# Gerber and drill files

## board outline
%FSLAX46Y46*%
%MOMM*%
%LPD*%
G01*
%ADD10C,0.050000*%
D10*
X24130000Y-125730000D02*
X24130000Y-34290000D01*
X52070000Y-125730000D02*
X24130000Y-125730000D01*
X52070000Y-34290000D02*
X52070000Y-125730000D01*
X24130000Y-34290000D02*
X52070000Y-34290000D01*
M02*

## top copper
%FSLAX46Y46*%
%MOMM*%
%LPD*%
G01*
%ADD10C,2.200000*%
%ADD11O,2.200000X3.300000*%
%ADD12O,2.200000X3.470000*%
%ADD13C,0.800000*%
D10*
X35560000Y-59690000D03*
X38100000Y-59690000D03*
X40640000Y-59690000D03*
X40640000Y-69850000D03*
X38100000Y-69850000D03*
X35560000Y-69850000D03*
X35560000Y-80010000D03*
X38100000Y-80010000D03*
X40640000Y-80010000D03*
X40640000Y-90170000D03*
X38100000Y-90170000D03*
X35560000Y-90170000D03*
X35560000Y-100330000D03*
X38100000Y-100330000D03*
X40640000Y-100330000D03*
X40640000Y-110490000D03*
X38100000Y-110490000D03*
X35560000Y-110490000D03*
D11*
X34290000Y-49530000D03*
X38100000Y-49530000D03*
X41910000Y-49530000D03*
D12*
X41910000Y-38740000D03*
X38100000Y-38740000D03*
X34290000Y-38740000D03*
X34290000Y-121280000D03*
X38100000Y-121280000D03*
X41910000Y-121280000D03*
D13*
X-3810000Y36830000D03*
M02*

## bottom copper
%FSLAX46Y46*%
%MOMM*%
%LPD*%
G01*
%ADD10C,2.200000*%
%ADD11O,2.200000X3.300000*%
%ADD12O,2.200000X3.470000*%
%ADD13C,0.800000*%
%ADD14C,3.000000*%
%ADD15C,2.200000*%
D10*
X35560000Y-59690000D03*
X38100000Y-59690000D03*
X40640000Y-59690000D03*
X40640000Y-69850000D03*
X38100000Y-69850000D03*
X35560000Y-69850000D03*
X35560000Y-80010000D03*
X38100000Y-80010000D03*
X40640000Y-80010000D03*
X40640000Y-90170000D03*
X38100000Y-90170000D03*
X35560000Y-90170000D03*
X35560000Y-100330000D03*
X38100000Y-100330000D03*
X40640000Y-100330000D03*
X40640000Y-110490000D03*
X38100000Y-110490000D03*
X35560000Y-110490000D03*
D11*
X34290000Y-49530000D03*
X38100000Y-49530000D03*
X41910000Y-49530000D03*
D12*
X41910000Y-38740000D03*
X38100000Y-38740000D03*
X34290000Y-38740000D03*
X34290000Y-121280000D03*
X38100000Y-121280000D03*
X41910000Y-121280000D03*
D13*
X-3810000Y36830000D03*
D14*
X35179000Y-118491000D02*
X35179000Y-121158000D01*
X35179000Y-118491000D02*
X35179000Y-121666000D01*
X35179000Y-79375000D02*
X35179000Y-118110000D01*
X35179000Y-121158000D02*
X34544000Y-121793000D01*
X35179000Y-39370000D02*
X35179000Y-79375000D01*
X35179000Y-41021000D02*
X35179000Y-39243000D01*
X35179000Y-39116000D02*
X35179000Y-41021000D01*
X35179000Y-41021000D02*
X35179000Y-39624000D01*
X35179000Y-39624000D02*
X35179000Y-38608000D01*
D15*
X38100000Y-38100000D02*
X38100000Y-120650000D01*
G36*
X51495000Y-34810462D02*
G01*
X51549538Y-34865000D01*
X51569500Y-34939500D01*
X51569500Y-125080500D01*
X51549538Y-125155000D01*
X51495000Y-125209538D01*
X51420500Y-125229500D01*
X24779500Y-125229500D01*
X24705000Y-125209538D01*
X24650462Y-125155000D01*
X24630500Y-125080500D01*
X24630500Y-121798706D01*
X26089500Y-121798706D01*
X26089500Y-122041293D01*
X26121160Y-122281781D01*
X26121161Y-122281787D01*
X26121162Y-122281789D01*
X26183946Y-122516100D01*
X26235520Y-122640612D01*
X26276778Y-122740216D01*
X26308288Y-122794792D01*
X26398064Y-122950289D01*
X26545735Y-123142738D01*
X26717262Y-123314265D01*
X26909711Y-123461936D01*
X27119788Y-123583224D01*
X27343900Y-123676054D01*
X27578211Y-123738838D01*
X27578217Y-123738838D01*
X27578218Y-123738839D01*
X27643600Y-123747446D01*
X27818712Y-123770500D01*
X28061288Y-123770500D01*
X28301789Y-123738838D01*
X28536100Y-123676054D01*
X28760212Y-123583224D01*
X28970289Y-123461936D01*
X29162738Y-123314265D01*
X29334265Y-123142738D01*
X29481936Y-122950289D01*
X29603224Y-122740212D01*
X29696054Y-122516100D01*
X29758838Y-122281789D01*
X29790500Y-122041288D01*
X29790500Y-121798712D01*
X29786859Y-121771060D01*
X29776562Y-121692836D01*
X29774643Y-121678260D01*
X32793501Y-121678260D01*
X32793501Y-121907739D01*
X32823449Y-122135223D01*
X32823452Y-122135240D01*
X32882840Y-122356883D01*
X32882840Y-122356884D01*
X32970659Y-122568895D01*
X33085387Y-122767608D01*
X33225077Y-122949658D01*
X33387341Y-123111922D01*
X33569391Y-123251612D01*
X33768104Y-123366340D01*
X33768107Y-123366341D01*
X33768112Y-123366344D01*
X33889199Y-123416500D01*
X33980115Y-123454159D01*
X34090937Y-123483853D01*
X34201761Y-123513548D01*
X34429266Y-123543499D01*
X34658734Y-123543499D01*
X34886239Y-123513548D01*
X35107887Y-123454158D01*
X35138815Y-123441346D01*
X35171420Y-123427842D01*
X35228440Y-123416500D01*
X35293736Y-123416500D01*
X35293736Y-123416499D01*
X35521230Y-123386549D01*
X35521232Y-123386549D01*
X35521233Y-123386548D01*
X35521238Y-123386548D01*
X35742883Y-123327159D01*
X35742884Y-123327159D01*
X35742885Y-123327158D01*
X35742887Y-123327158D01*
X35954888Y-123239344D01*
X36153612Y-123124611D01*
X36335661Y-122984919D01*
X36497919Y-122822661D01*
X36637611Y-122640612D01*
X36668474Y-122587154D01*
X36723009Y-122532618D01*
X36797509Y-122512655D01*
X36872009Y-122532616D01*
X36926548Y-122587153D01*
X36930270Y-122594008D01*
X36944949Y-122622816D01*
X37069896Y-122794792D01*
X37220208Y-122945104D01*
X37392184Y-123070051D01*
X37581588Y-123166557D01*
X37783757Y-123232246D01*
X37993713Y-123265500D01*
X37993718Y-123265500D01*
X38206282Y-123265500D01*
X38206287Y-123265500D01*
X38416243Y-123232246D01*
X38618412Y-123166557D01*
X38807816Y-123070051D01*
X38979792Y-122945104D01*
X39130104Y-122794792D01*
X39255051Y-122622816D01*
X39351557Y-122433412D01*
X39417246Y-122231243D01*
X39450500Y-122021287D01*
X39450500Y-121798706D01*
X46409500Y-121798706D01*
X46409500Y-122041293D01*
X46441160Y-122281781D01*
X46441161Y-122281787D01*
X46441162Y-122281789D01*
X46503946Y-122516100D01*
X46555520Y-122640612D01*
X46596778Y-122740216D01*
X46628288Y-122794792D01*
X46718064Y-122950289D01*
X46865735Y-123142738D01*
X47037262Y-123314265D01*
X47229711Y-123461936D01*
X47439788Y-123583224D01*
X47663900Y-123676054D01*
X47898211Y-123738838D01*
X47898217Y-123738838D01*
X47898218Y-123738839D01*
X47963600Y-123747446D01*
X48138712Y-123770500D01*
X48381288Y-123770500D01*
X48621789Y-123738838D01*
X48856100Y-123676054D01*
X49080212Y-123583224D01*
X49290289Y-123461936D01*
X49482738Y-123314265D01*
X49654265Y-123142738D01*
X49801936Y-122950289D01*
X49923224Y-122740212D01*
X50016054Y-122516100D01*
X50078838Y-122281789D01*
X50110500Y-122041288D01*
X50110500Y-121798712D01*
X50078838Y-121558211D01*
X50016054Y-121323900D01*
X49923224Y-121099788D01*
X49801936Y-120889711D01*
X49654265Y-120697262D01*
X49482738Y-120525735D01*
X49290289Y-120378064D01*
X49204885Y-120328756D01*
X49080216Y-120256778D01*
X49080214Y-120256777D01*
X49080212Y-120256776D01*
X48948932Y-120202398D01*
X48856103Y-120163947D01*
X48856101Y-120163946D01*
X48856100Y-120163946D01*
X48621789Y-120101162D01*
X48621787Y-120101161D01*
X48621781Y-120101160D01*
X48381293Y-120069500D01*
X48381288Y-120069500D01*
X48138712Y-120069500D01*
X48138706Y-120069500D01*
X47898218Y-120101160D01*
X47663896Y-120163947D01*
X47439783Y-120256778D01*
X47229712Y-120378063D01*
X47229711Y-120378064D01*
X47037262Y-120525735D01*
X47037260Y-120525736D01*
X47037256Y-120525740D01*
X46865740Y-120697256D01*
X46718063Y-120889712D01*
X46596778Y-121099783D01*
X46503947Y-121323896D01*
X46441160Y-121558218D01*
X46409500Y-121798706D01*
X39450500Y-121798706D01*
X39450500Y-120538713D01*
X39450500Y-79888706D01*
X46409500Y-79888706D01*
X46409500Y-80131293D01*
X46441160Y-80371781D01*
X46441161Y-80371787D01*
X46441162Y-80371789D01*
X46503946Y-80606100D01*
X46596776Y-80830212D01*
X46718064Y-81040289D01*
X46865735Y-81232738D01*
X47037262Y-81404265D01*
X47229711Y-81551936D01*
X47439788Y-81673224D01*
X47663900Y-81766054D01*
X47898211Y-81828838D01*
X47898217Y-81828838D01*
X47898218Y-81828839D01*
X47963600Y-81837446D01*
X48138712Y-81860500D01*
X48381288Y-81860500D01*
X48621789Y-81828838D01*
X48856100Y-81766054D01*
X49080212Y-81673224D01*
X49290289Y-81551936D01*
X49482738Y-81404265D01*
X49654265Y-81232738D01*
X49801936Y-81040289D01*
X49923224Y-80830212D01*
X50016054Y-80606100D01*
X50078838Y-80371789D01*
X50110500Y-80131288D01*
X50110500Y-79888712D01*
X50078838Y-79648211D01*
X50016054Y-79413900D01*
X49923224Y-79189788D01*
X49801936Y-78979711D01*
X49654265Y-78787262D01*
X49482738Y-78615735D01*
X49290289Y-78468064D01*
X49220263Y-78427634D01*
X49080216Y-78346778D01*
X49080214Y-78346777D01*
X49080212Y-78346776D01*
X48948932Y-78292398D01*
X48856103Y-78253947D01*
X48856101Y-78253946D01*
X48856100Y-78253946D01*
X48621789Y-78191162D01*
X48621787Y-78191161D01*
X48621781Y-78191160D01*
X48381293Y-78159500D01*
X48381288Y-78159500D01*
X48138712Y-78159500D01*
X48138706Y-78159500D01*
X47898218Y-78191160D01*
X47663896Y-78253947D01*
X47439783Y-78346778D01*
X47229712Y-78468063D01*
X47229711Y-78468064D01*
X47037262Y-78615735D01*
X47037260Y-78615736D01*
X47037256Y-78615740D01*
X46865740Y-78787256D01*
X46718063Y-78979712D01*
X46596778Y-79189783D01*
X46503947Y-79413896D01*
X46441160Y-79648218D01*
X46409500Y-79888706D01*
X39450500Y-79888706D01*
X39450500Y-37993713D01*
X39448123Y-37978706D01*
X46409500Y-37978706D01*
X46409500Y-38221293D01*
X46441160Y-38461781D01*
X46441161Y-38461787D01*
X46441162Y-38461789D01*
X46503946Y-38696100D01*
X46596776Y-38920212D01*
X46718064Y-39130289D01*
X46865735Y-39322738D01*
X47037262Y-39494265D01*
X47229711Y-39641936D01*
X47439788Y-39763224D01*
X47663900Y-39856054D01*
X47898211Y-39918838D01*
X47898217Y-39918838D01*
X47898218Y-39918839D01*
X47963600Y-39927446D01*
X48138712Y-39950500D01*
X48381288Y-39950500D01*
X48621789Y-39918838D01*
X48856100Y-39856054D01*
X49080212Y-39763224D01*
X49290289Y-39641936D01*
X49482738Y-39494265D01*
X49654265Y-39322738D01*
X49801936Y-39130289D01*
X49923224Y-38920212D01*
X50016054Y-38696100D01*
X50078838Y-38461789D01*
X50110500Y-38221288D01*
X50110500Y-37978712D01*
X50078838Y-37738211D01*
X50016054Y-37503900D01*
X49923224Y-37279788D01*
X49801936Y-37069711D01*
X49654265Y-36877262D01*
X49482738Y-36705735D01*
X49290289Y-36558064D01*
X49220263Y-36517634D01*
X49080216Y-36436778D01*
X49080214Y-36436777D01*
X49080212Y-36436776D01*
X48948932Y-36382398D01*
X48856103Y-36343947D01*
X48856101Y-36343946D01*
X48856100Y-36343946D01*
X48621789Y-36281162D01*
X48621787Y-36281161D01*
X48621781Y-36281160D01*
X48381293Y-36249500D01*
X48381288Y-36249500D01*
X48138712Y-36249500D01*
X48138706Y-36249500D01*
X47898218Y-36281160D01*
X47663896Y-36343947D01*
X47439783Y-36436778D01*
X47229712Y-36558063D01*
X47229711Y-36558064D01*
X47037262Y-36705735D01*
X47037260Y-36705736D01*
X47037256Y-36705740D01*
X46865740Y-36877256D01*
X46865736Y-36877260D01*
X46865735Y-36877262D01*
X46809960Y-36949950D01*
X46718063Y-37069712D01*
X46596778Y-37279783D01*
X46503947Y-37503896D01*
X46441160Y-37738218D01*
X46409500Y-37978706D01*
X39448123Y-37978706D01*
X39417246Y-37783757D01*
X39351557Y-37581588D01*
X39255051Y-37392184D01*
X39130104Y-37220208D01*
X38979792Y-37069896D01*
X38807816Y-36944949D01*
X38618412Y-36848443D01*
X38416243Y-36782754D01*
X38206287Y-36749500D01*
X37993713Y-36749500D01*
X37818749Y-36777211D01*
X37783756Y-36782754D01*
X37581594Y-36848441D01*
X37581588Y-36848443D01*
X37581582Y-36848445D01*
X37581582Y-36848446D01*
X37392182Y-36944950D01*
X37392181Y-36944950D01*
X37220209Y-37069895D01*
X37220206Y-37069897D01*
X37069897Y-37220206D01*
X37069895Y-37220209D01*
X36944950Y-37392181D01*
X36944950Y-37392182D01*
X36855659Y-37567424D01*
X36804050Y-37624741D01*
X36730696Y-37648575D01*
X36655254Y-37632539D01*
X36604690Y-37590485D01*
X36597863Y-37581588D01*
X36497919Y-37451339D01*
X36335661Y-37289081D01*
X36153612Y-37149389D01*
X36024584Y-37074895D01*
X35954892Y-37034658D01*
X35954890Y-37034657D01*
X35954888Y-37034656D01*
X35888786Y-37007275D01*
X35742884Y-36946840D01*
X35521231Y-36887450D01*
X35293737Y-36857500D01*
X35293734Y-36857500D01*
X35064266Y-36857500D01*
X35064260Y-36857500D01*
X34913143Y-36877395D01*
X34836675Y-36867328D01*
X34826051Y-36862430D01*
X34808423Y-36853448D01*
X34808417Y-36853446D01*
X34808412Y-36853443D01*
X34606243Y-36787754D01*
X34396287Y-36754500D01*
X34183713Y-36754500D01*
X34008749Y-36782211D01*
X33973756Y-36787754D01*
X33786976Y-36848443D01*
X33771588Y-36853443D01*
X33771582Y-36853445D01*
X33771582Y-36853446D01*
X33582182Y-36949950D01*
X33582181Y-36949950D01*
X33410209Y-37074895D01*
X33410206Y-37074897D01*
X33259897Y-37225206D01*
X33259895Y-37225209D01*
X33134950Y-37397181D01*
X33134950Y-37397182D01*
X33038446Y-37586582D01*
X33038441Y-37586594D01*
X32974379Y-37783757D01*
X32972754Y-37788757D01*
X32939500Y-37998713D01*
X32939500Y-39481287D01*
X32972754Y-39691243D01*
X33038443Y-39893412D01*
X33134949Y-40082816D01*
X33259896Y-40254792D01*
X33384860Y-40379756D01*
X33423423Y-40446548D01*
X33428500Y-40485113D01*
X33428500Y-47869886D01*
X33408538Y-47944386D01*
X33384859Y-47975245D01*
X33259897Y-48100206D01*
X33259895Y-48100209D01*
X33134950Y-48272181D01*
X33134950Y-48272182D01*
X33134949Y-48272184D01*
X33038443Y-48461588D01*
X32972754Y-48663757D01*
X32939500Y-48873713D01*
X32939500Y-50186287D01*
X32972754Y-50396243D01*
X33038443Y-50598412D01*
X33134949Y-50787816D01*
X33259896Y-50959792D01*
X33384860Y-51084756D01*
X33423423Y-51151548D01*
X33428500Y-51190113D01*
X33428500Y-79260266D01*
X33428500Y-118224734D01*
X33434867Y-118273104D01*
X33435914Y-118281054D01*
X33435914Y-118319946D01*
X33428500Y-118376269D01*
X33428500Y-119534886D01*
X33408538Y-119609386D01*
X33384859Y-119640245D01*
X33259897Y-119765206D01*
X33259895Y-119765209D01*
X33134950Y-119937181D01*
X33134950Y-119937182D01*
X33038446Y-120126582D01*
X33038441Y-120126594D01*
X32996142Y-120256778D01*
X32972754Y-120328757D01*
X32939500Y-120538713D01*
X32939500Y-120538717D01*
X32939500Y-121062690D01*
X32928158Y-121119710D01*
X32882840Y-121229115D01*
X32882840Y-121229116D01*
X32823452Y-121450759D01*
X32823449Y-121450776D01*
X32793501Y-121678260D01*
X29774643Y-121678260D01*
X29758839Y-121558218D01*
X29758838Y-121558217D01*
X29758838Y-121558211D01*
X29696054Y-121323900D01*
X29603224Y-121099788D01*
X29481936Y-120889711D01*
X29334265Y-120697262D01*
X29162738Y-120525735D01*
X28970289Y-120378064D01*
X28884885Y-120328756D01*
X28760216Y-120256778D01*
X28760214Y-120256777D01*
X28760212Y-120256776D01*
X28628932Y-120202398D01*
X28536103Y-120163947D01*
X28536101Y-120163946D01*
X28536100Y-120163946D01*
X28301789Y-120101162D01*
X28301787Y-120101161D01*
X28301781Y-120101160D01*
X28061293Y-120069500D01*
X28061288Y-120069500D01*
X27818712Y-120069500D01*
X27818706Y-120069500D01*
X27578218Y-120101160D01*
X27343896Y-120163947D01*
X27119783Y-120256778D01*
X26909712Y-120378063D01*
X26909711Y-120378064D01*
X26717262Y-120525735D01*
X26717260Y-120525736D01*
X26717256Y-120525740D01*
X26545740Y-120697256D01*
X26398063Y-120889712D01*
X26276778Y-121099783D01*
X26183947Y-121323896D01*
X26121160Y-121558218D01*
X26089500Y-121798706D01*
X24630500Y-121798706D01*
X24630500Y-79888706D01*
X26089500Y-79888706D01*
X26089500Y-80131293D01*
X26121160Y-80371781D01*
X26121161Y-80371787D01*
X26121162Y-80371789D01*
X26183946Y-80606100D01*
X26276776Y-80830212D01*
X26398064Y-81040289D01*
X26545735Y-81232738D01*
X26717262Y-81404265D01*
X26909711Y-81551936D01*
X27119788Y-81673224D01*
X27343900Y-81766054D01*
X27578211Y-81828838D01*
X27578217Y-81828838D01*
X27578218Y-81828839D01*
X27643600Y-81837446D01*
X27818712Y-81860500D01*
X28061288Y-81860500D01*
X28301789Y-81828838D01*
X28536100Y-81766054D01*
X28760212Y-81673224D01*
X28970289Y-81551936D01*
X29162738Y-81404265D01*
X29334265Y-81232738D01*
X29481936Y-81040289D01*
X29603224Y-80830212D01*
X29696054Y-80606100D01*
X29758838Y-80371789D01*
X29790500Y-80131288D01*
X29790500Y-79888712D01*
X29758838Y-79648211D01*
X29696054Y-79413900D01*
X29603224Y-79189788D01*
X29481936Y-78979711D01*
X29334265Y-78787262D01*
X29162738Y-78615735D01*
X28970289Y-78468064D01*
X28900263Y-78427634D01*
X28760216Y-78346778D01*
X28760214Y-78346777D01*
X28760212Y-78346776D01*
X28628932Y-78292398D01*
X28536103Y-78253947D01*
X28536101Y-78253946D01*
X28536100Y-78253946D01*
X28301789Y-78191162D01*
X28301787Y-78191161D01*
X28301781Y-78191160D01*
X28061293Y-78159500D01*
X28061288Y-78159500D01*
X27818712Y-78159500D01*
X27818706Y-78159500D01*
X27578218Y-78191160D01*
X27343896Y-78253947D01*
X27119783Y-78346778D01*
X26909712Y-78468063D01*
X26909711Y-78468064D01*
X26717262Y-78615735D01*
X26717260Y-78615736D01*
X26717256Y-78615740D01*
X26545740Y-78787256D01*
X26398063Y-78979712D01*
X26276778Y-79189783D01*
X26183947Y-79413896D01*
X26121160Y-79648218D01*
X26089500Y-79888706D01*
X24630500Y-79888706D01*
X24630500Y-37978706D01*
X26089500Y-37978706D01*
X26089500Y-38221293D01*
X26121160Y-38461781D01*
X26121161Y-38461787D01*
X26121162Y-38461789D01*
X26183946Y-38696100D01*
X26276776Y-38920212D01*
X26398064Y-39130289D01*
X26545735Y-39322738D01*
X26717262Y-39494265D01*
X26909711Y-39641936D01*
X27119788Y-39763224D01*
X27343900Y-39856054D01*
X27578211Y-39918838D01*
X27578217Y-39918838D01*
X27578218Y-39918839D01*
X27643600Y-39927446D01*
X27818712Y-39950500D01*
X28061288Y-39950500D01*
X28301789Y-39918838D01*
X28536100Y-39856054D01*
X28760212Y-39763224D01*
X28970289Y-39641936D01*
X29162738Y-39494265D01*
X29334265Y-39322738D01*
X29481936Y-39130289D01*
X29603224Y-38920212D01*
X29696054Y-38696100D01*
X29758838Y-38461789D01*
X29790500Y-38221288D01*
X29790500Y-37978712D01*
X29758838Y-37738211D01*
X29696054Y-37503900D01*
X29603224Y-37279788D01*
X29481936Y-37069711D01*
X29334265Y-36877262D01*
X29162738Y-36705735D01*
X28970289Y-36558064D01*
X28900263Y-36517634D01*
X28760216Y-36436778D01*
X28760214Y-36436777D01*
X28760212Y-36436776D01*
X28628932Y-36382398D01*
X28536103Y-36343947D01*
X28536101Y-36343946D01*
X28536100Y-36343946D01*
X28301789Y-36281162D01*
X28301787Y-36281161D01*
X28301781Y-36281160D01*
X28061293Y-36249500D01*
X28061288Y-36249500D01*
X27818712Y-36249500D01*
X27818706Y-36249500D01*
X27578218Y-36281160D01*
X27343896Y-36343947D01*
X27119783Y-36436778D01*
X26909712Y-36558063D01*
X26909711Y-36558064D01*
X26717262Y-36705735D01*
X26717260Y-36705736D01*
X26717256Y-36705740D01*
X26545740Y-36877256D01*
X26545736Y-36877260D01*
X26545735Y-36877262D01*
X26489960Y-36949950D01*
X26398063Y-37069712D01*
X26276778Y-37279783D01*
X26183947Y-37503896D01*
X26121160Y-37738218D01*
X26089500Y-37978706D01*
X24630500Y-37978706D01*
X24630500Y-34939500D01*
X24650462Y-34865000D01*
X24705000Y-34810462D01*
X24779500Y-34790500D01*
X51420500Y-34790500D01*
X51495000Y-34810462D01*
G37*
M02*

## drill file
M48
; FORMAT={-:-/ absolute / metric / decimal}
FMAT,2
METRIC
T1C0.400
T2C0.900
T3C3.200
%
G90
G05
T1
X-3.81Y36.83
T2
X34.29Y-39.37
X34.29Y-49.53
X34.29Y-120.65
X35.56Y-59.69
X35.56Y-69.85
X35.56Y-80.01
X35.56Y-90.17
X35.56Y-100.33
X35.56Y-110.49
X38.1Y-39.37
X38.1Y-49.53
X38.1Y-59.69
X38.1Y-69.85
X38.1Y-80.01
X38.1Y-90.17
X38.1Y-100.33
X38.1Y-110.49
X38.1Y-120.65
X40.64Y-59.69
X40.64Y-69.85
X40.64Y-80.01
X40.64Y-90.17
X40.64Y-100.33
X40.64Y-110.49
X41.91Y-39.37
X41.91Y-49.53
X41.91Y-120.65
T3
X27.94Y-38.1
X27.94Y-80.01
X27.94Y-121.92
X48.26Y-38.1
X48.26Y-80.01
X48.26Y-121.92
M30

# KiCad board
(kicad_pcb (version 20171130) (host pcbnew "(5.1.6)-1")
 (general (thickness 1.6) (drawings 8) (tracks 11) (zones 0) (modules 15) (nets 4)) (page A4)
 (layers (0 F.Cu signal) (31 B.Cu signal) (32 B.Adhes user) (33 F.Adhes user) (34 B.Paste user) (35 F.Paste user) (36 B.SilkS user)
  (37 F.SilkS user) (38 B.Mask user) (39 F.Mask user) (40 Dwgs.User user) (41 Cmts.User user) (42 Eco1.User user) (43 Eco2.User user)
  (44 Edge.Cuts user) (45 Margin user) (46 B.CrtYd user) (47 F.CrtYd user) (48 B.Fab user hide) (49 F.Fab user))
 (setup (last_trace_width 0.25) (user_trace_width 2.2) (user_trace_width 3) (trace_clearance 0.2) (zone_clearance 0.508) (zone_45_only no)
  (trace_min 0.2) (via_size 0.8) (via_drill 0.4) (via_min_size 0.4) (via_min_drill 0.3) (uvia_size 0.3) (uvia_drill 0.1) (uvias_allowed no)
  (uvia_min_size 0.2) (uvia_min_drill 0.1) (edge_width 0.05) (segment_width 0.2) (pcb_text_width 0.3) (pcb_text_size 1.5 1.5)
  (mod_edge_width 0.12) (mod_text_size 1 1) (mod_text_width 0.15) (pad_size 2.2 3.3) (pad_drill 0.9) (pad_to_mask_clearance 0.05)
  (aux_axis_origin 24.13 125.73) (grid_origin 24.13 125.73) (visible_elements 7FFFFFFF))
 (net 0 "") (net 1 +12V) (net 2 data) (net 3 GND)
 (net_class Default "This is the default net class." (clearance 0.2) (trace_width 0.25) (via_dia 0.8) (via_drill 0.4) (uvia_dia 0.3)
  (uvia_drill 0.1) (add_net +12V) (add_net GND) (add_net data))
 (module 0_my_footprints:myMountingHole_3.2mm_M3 (layer F.Cu) (at 48.26 80.01)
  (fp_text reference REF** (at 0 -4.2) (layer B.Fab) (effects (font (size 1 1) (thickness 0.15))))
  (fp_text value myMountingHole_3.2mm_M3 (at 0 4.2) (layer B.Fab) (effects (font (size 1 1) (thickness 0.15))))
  (pad "" np_thru_hole circle (at 0 0) (size 3.2 3.2) (drill 3.2) (layers *.Cu *.Mask)))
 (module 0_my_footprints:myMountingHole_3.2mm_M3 (layer F.Cu) (at 27.94 80.01)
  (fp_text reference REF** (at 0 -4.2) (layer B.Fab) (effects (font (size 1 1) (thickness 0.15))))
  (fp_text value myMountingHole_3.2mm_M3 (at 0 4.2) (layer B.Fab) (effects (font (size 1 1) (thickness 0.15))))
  (pad "" np_thru_hole circle (at 0 0) (size 3.2 3.2) (drill 3.2) (layers *.Cu *.Mask)))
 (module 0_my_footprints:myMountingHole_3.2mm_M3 (layer F.Cu) (at 27.94 121.92)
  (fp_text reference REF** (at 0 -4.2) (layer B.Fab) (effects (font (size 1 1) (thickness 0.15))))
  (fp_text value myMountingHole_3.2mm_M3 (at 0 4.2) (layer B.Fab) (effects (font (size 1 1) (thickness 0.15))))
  (pad "" np_thru_hole circle (at 0 0) (size 3.2 3.2) (drill 3.2) (layers *.Cu *.Mask)))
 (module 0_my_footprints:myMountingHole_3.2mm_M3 (layer F.Cu) (at 48.26 121.92)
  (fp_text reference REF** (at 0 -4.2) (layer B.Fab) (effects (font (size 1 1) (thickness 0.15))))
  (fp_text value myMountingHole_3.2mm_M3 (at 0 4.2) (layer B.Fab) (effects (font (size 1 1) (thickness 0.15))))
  (pad "" np_thru_hole circle (at 0 0) (size 3.2 3.2) (drill 3.2) (layers *.Cu *.Mask)))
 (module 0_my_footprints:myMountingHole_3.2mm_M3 (layer F.Cu) (at 27.94 38.1)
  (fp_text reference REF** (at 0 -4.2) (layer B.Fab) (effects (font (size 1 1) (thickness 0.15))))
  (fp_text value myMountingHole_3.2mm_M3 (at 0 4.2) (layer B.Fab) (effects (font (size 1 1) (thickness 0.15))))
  (pad "" np_thru_hole circle (at 0 0) (size 3.2 3.2) (drill 3.2) (layers *.Cu *.Mask)))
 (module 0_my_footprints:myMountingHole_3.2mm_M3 (layer F.Cu) (at 48.26 38.1)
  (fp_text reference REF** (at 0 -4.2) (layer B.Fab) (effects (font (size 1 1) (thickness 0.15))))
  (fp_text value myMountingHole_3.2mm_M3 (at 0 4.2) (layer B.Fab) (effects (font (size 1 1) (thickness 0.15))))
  (pad "" np_thru_hole circle (at 0 0) (size 3.2 3.2) (drill 3.2) (layers *.Cu *.Mask)))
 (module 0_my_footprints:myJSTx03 (layer F.Cu) (at 35.56 59.69)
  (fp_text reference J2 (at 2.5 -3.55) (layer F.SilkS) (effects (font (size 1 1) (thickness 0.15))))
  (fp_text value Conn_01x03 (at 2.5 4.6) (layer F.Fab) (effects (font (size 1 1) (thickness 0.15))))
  (pad 1 thru_hole circle (at 0 0) (size 2.2 2.2) (drill 0.9) (layers *.Cu *.Mask) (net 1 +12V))
  (pad 2 thru_hole circle (at 2.54 0) (size 2.2 2.2) (drill 0.9) (layers *.Cu *.Mask) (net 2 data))
  (pad 3 thru_hole circle (at 5.08 0) (size 2.2 2.2) (drill 0.9) (layers *.Cu *.Mask) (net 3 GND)))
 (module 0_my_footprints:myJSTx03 (layer F.Cu) (at 35.56 69.85)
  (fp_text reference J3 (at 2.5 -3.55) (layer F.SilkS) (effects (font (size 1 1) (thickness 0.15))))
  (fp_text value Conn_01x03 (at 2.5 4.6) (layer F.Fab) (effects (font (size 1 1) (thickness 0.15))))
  (pad 3 thru_hole circle (at 5.08 0) (size 2.2 2.2) (drill 0.9) (layers *.Cu *.Mask) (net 3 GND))
  (pad 2 thru_hole circle (at 2.54 0) (size 2.2 2.2) (drill 0.9) (layers *.Cu *.Mask) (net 2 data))
  (pad 1 thru_hole circle (at 0 0) (size 2.2 2.2) (drill 0.9) (layers *.Cu *.Mask) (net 1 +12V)))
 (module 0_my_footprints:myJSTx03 (layer F.Cu) (at 35.56 80.01)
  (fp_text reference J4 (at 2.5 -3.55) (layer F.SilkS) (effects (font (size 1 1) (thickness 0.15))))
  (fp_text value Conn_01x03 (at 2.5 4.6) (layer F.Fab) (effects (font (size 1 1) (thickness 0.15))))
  (pad 1 thru_hole circle (at 0 0) (size 2.2 2.2) (drill 0.9) (layers *.Cu *.Mask) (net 1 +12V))
  (pad 2 thru_hole circle (at 2.54 0) (size 2.2 2.2) (drill 0.9) (layers *.Cu *.Mask) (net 2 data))
  (pad 3 thru_hole circle (at 5.08 0) (size 2.2 2.2) (drill 0.9) (layers *.Cu *.Mask) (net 3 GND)))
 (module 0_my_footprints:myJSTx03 (layer F.Cu) (at 35.56 90.17)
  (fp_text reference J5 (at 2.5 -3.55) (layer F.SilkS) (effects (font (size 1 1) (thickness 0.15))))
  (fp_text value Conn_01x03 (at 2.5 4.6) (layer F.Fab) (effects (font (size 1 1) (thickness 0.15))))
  (pad 3 thru_hole circle (at 5.08 0) (size 2.2 2.2) (drill 0.9) (layers *.Cu *.Mask) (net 3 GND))
  (pad 2 thru_hole circle (at 2.54 0) (size 2.2 2.2) (drill 0.9) (layers *.Cu *.Mask) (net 2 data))
  (pad 1 thru_hole circle (at 0 0) (size 2.2 2.2) (drill 0.9) (layers *.Cu *.Mask) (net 1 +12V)))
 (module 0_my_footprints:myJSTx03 (layer F.Cu) (at 35.56 100.33)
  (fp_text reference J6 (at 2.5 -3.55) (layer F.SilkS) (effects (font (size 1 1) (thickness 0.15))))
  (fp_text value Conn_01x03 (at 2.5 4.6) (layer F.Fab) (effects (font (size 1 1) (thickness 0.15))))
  (pad 1 thru_hole circle (at 0 0) (size 2.2 2.2) (drill 0.9) (layers *.Cu *.Mask) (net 1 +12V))
  (pad 2 thru_hole circle (at 2.54 0) (size 2.2 2.2) (drill 0.9) (layers *.Cu *.Mask) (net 2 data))
  (pad 3 thru_hole circle (at 5.08 0) (size 2.2 2.2) (drill 0.9) (layers *.Cu *.Mask) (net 3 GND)))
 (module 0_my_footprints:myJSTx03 (layer F.Cu) (at 35.56 110.49)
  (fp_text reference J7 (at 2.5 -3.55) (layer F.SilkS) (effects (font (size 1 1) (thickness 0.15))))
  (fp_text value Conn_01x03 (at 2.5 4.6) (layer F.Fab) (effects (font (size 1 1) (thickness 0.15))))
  (pad 3 thru_hole circle (at 5.08 0) (size 2.2 2.2) (drill 0.9) (layers *.Cu *.Mask) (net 3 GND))
  (pad 2 thru_hole circle (at 2.54 0) (size 2.2 2.2) (drill 0.9) (layers *.Cu *.Mask) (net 2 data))
  (pad 1 thru_hole circle (at 0 0) (size 2.2 2.2) (drill 0.9) (layers *.Cu *.Mask) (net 1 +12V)))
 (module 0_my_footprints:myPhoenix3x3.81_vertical (layer F.Cu) (at 34.29 49.53)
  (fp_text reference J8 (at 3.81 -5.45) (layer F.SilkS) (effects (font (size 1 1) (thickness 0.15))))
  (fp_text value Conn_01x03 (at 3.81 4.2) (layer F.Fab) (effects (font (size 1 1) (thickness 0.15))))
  (pad 1 thru_hole oval (at 0 0) (size 2.2 3.3) (drill 0.9) (layers *.Cu *.Mask) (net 1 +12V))
  (pad 2 thru_hole oval (at 3.81 0) (size 2.2 3.3) (drill 0.9) (layers *.Cu *.Mask) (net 2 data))
  (pad 3 thru_hole oval (at 7.62 0) (size 2.2 3.3) (drill 0.9) (layers *.Cu *.Mask) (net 3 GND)))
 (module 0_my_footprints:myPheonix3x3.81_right (layer F.Cu) (at 41.91 39.37 180)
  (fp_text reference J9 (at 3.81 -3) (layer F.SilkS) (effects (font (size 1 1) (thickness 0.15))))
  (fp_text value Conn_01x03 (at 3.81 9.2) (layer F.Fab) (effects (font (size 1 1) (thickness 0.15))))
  (pad 1 thru_hole oval (at 0 0 180) (size 2.2 3.47) (drill 0.9 (offset 0 0.63)) (layers *.Cu *.Mask) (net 3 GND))
  (pad 2 thru_hole oval (at 3.81 0 180) (size 2.2 3.47) (drill 0.9 (offset 0 0.63)) (layers *.Cu *.Mask) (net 2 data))
  (pad 3 thru_hole oval (at 7.62 0 180) (size 2.2 3.47) (drill 0.9 (offset 0 0.63)) (layers *.Cu *.Mask) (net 1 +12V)))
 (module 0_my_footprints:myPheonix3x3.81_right (layer F.Cu) (at 34.29 120.65)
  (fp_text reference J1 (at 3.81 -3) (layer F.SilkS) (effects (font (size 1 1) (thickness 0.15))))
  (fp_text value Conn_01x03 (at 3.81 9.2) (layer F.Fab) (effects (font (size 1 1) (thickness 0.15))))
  (pad 1 thru_hole oval (at 0 0) (size 2.2 3.47) (drill 0.9 (offset 0 0.63)) (layers *.Cu *.Mask) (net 1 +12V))
  (pad 2 thru_hole oval (at 3.81 0) (size 2.2 3.47) (drill 0.9 (offset 0 0.63)) (layers *.Cu *.Mask) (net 2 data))
  (pad 3 thru_hole oval (at 7.62 0) (size 2.2 3.47) (drill 0.9 (offset 0 0.63)) (layers *.Cu *.Mask) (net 3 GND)))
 (gr_line (start 24.13 125.73) (end 24.13 34.29) (layer Edge.Cuts) (width 0.05))
 (gr_line (start 52.07 125.73) (end 24.13 125.73) (layer Edge.Cuts) (width 0.05))
 (gr_line (start 52.07 34.29) (end 52.07 125.73) (layer Edge.Cuts) (width 0.05))
 (gr_line (start 24.13 34.29) (end 52.07 34.29) (layer Edge.Cuts) (width 0.05))
 (via (at -3.81 -36.83) (size 0.8) (drill 0.4) (layers F.Cu B.Cu) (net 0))
 (segment (start 35.179 118.491) (end 35.179 121.158) (width 3) (layer B.Cu) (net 1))
 (segment (start 35.179 118.491) (end 35.179 121.666) (width 3) (layer B.Cu) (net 1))
 (segment (start 35.179 79.375) (end 35.179 118.11) (width 3) (layer B.Cu) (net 1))
 (segment (start 35.179 121.158) (end 34.544 121.793) (width 3) (layer B.Cu) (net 1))
 (segment (start 35.179 39.37) (end 35.179 79.375) (width 3) (layer B.Cu) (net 1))
 (segment (start 35.179 41.021) (end 35.179 39.243) (width 3) (layer B.Cu) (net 1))
 (segment (start 35.179 39.116) (end 35.179 41.021) (width 3) (layer B.Cu) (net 1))
 (segment (start 35.179 41.021) (end 35.179 39.624) (width 3) (layer B.Cu) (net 1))
 (segment (start 35.179 39.624) (end 35.179 38.608) (width 3) (layer B.Cu) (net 1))
 (segment (start 38.1 38.1) (end 38.1 120.65) (width 2.2) (layer B.Cu) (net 2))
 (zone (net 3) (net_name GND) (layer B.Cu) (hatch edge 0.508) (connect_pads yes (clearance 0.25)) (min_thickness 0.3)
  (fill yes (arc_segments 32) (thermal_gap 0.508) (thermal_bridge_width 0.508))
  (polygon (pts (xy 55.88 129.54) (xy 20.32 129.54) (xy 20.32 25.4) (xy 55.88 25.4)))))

